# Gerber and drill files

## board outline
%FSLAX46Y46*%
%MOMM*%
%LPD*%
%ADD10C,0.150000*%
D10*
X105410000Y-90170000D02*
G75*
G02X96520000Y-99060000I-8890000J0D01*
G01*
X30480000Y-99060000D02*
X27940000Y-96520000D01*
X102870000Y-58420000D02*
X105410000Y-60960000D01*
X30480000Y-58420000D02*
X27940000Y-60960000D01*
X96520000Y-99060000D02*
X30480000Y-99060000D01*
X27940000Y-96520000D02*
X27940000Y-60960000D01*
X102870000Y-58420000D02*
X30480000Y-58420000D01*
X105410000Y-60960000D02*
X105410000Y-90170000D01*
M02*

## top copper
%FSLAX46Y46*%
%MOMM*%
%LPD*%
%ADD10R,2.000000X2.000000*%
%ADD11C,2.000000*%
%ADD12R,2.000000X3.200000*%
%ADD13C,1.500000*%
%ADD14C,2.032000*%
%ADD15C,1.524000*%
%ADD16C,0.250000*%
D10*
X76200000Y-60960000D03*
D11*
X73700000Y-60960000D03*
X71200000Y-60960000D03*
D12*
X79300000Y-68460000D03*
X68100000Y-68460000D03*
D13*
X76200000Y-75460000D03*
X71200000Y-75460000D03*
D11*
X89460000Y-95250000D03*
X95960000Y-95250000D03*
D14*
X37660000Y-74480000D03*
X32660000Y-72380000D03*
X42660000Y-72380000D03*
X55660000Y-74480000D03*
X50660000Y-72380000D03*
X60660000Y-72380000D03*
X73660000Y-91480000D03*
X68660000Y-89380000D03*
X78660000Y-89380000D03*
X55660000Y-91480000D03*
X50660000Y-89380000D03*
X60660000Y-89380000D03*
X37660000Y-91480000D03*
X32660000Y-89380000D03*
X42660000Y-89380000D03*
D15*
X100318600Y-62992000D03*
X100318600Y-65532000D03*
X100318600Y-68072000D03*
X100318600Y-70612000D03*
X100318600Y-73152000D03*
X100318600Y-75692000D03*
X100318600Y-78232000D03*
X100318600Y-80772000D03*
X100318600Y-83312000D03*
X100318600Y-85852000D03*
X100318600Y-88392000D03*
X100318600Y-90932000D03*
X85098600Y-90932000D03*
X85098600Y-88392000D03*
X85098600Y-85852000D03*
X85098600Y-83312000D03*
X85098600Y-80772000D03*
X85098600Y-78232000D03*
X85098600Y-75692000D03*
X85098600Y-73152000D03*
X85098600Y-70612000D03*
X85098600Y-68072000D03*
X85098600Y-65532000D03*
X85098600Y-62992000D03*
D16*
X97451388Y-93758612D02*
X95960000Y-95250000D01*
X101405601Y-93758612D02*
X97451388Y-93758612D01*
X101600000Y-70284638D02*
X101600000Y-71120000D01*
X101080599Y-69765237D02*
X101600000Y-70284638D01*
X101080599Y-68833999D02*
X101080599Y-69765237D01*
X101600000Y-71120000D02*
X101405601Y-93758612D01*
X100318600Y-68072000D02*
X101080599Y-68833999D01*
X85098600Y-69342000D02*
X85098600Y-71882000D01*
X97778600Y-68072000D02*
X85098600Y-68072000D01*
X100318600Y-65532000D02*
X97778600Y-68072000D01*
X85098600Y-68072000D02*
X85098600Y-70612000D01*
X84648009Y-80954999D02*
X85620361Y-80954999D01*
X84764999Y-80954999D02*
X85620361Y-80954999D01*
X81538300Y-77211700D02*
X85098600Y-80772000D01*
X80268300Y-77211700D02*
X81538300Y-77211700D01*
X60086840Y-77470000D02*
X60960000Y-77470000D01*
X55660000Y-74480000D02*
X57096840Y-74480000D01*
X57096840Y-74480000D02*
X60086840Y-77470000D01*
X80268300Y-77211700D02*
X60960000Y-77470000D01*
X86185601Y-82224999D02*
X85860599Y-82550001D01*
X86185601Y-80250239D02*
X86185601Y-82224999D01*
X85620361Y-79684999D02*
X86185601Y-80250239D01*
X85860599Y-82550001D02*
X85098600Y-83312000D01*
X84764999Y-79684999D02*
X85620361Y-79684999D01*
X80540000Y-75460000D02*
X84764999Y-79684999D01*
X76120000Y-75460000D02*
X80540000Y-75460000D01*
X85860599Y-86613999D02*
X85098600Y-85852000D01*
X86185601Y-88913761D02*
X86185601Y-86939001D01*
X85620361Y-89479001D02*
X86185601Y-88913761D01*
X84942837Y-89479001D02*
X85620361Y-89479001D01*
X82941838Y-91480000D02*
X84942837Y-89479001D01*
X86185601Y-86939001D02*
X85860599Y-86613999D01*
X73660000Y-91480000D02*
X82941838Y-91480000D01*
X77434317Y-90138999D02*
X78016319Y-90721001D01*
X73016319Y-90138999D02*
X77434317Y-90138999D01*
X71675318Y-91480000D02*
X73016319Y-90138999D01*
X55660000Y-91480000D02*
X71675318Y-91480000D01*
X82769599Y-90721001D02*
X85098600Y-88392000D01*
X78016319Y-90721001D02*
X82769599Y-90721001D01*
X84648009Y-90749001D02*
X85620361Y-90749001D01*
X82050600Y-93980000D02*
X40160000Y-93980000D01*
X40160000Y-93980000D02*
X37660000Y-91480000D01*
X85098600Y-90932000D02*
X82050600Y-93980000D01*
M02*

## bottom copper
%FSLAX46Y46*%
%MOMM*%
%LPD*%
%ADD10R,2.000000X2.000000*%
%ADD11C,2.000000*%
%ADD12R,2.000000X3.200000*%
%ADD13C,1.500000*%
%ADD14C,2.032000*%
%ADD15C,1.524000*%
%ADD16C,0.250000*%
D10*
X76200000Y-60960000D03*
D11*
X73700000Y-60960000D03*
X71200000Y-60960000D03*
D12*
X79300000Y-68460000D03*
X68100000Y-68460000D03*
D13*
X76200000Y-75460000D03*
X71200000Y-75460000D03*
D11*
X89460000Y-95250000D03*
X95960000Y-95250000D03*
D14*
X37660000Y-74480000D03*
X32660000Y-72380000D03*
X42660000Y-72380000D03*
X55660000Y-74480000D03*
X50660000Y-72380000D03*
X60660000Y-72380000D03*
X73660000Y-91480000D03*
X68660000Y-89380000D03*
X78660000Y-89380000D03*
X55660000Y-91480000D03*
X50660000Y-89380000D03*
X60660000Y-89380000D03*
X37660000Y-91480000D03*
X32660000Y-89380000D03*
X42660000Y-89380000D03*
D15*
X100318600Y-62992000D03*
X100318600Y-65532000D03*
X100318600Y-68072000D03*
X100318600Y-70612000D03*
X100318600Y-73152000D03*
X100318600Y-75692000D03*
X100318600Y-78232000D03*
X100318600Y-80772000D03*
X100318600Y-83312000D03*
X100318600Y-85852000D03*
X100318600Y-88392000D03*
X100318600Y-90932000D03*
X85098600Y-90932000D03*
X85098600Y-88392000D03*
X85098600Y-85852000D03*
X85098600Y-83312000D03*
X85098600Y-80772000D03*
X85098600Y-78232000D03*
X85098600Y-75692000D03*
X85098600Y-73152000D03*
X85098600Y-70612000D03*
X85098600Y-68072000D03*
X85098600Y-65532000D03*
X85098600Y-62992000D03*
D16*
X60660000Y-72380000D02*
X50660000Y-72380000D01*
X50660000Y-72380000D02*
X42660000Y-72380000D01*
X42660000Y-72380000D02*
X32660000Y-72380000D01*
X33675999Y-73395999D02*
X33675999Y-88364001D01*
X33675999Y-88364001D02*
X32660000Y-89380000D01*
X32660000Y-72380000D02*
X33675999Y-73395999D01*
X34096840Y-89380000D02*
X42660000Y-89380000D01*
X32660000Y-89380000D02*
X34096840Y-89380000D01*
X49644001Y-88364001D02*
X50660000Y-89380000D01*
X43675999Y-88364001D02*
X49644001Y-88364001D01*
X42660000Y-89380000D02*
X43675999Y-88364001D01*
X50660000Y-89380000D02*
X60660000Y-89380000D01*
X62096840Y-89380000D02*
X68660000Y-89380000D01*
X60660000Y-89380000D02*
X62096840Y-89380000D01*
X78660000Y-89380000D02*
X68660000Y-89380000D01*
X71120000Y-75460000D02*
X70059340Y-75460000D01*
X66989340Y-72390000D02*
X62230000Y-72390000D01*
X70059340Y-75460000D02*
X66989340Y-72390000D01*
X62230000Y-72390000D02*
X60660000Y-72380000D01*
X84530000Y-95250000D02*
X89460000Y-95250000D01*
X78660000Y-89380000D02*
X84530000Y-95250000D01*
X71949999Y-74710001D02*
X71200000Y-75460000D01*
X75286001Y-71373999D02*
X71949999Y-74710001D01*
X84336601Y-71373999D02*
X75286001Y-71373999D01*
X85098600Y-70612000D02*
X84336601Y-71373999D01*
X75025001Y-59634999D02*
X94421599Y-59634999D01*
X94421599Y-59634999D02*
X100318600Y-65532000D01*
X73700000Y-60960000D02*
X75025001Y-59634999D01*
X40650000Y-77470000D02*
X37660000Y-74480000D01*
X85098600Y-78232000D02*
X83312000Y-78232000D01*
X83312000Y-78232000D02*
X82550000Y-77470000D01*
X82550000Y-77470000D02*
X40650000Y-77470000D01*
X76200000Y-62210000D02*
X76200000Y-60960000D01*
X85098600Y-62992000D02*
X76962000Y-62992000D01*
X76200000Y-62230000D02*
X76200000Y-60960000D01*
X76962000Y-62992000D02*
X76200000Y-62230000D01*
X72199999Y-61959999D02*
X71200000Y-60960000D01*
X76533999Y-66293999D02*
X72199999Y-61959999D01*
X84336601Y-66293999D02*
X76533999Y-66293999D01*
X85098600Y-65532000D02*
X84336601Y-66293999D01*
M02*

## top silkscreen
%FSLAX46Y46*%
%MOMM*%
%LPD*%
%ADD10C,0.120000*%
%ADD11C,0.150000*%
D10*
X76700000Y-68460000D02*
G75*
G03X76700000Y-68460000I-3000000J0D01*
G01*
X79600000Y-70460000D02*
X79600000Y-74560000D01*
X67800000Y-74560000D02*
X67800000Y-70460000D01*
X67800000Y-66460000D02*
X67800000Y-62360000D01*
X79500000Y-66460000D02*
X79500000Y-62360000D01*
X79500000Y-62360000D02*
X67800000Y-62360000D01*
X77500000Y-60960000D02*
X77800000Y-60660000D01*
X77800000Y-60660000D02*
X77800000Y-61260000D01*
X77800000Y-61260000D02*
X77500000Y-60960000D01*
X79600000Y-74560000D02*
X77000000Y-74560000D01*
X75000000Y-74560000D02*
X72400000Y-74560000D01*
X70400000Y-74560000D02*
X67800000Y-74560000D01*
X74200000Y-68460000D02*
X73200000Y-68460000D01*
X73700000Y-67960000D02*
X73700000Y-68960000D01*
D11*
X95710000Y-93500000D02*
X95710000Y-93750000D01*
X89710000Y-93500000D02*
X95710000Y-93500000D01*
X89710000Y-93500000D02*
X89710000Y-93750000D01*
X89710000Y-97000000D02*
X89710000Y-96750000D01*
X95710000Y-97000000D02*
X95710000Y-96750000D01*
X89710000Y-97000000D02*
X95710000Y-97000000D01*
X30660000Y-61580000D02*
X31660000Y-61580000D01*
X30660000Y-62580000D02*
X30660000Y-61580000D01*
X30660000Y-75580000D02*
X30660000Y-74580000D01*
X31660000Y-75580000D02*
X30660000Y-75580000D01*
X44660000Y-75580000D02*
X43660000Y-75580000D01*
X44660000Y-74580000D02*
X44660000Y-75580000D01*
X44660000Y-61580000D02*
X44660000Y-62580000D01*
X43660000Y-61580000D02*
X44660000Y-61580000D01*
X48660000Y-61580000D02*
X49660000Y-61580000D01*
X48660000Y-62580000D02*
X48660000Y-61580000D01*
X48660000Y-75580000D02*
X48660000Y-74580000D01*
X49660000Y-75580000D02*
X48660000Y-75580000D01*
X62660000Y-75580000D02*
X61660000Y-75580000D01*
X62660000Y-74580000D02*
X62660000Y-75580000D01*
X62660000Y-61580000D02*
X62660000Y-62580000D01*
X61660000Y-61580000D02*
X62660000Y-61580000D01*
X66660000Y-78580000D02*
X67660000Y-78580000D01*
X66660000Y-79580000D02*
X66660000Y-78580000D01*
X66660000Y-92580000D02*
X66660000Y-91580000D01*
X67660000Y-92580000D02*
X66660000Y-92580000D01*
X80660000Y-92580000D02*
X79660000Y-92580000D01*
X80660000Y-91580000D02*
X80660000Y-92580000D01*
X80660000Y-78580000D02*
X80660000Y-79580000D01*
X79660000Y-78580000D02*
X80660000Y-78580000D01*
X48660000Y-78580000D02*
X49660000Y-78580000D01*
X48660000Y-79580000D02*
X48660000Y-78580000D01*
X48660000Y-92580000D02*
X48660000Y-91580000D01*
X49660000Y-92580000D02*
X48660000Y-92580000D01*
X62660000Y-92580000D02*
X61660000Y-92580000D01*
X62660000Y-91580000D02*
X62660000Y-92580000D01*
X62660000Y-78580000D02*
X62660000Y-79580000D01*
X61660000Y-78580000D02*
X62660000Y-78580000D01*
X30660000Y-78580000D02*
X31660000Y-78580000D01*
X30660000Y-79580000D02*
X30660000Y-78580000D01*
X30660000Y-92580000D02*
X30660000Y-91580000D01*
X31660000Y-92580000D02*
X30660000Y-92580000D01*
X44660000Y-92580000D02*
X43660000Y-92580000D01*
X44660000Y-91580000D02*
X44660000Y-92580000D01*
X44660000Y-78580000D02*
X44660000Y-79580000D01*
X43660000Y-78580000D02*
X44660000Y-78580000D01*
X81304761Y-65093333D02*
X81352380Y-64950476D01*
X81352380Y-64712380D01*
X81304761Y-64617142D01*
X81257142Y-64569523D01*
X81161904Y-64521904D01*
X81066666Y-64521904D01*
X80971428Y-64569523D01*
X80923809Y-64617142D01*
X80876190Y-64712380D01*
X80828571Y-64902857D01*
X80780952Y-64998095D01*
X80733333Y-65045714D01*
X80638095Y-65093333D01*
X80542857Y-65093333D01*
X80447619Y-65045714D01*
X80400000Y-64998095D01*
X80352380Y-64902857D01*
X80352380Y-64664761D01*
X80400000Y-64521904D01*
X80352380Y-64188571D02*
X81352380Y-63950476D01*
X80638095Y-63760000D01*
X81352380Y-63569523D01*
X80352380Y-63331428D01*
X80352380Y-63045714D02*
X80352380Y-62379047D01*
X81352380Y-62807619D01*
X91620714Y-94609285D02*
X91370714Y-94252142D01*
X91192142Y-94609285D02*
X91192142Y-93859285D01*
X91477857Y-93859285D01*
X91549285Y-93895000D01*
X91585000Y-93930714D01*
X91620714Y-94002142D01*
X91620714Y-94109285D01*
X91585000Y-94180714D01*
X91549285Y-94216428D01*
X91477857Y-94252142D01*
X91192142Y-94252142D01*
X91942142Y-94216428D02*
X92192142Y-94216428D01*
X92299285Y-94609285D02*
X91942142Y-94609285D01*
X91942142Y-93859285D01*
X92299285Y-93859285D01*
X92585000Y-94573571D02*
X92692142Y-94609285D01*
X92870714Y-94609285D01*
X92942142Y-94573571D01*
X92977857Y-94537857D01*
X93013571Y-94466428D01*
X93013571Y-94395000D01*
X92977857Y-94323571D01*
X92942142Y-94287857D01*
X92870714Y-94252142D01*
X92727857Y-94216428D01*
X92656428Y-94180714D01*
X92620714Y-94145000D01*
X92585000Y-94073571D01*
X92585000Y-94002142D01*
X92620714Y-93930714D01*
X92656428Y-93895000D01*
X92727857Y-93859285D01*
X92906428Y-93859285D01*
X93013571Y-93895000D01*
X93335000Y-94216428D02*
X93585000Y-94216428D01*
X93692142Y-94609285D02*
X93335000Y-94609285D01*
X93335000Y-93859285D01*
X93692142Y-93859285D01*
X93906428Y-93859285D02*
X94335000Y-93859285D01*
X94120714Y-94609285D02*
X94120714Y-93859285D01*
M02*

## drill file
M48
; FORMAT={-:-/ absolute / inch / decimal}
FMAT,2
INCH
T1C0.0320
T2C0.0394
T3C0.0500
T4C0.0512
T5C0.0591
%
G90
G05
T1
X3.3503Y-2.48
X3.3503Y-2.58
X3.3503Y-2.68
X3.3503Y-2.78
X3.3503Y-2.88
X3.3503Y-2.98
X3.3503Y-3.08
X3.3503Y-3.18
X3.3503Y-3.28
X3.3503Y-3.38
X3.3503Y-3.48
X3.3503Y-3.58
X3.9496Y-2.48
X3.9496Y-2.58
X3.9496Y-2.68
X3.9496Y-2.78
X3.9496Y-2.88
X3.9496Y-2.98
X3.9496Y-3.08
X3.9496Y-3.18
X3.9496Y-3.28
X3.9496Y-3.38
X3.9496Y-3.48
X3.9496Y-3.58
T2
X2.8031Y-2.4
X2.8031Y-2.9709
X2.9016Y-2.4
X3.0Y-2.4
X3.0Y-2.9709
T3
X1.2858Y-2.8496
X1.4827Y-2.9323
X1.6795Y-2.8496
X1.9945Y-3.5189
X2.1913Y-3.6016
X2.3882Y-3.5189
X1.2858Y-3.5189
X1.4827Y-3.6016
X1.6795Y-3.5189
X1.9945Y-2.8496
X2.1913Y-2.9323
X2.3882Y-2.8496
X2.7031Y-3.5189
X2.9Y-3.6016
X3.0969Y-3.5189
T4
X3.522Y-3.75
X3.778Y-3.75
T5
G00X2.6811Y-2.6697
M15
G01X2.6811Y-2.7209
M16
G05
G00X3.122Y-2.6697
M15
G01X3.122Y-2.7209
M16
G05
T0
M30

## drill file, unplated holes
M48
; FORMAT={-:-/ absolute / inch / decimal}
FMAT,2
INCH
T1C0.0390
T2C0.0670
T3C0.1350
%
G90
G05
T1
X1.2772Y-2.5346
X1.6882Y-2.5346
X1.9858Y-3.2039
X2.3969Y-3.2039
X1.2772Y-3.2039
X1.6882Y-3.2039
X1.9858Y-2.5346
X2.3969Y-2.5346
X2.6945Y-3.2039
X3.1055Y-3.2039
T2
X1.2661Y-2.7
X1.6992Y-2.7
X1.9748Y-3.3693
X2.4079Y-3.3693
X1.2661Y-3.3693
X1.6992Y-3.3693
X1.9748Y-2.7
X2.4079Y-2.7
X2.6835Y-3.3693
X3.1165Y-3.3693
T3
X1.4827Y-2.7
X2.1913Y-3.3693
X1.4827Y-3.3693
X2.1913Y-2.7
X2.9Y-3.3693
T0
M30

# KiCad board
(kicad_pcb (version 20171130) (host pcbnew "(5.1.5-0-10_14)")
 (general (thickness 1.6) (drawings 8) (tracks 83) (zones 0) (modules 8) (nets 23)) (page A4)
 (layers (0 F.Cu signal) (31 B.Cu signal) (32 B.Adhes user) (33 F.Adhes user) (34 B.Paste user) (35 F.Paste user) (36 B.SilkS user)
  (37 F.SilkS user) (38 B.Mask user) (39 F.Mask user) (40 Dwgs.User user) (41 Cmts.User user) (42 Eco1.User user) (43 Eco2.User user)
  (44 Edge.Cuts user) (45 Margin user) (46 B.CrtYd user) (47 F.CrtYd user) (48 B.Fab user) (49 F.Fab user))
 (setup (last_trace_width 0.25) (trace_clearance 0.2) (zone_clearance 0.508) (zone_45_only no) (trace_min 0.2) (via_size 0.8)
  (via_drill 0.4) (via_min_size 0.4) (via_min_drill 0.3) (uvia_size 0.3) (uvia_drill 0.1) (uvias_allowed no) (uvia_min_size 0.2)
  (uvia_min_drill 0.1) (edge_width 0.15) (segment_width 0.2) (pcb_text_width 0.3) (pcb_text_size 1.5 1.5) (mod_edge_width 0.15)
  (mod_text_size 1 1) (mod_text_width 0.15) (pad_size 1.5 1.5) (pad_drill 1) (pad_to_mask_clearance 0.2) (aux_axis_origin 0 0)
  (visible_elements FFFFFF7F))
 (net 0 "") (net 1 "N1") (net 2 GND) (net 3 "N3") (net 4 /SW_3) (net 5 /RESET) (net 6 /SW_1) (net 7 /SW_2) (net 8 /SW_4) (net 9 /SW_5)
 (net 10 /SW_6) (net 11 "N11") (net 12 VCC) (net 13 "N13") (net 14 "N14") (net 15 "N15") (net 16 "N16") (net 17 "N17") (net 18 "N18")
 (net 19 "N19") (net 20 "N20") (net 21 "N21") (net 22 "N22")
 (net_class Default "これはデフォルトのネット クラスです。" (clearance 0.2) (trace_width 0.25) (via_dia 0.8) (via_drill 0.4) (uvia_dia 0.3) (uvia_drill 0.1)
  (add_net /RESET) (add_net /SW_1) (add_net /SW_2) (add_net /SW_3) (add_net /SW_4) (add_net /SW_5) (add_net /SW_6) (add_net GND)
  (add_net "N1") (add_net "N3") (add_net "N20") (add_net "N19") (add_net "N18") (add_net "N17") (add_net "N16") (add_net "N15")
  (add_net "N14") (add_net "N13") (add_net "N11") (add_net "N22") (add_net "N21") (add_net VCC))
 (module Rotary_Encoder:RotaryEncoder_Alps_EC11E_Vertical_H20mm (layer F.Cu) (at 76.2 60.96 270)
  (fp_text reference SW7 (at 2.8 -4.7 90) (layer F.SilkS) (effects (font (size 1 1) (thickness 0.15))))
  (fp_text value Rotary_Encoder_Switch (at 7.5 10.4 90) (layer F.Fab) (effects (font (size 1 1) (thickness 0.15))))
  (fp_circle (center 7.5 2.5) (end 10.5 2.5) (layer F.SilkS) (width 0.12))
  (fp_line (start 9.5 -3.4) (end 13.6 -3.4) (layer F.SilkS) (width 0.12))
  (fp_line (start 13.6 8.4) (end 9.5 8.4) (layer F.SilkS) (width 0.12))
  (fp_line (start 5.5 8.4) (end 1.4 8.4) (layer F.SilkS) (width 0.12))
  (fp_line (start 5.5 -3.3) (end 1.4 -3.3) (layer F.SilkS) (width 0.12))
  (fp_line (start 1.4 -3.3) (end 1.4 8.4) (layer F.SilkS) (width 0.12))
  (fp_line (start 0 -1.3) (end -0.3 -1.6) (layer F.SilkS) (width 0.12))
  (fp_line (start -0.3 -1.6) (end 0.3 -1.6) (layer F.SilkS) (width 0.12))
  (fp_line (start 0.3 -1.6) (end 0 -1.3) (layer F.SilkS) (width 0.12))
  (fp_line (start 13.6 -3.4) (end 13.6 -0.8) (layer F.SilkS) (width 0.12))
  (fp_line (start 13.6 1.2) (end 13.6 3.8) (layer F.SilkS) (width 0.12))
  (fp_line (start 13.6 5.8) (end 13.6 8.4) (layer F.SilkS) (width 0.12))
  (fp_line (start 7.5 2) (end 7.5 3) (layer F.SilkS) (width 0.12))
  (fp_line (start 7 2.5) (end 8 2.5) (layer F.SilkS) (width 0.12))
  (pad A thru_hole rect (at 0 0 270) (size 2 2) (drill 1) (layers *.Cu *.Mask) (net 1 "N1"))
  (pad C thru_hole circle (at 0 2.5 270) (size 2 2) (drill 1) (layers *.Cu *.Mask) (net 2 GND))
  (pad B thru_hole circle (at 0 5 270) (size 2 2) (drill 1) (layers *.Cu *.Mask) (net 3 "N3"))
  (pad MP thru_hole rect (at 7.5 -3.1 270) (size 3.2 2) (drill oval 2.8 1.5) (layers *.Cu *.Mask))
  (pad MP thru_hole rect (at 7.5 8.1 270) (size 3.2 2) (drill oval 2.8 1.5) (layers *.Cu *.Mask))
  (pad "" thru_hole circle (at 14.5 0 270) (size 1.5 1.5) (drill 1) (layers *.Cu *.Mask) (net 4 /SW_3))
  (pad "" thru_hole circle (at 14.5 5 270) (size 1.5 1.5) (drill 1) (layers *.Cu *.Mask) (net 2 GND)))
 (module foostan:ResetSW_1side (layer F.Cu) (at 92.71 95.25)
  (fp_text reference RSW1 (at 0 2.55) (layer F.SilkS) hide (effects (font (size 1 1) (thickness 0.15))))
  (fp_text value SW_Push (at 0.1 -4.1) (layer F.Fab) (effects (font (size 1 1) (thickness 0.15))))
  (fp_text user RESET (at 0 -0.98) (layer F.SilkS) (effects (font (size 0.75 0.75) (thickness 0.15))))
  (fp_line (start 3 -1.75) (end 3 -1.5) (layer F.SilkS) (width 0.15))
  (fp_line (start -3 -1.75) (end 3 -1.75) (layer F.SilkS) (width 0.15))
  (fp_line (start -3 -1.75) (end -3 -1.5) (layer F.SilkS) (width 0.15))
  (fp_line (start -3 1.75) (end -3 1.5) (layer F.SilkS) (width 0.15))
  (fp_line (start 3 1.75) (end 3 1.5) (layer F.SilkS) (width 0.15))
  (fp_line (start -3 1.75) (end 3 1.75) (layer F.SilkS) (width 0.15))
  (pad 2 thru_hole circle (at -3.25 0) (size 2 2) (drill 1.3) (layers *.Cu F.SilkS B.Mask) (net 2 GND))
  (pad 1 thru_hole circle (at 3.25 0) (size 2 2) (drill 1.3) (layers *.Cu F.SilkS B.Mask) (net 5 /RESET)))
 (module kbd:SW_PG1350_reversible (layer F.Cu) (at 37.66 68.58)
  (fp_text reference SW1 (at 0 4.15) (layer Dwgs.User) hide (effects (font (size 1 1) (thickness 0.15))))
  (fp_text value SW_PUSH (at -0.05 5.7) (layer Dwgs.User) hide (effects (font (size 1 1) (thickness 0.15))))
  (fp_line (start -7 -7) (end -6 -7) (layer F.SilkS) (width 0.15))
  (fp_line (start -7 -6) (end -7 -7) (layer F.SilkS) (width 0.15))
  (fp_line (start -7 7) (end -7 6) (layer F.SilkS) (width 0.15))
  (fp_line (start -6 7) (end -7 7) (layer F.SilkS) (width 0.15)) (fp_line (start 7 7) (end 6 7) (layer F.SilkS) (width 0.15))
  (fp_line (start 7 6) (end 7 7) (layer F.SilkS) (width 0.15))
  (fp_line (start 7 -7) (end 7 -6) (layer F.SilkS) (width 0.15))
  (fp_line (start 6 -7) (end 7 -7) (layer F.SilkS) (width 0.15))
  (pad "" np_thru_hole circle (at -5.5 0) (size 1.7018 1.7018) (drill 1.7018) (layers *.Cu *.Mask))
  (pad "" np_thru_hole circle (at 5.5 0) (size 1.7018 1.7018) (drill 1.7018) (layers *.Cu *.Mask))
  (pad "" np_thru_hole circle (at 5.22 -4.2) (size 0.9906 0.9906) (drill 0.9906) (layers *.Cu *.Mask))
  (pad 1 thru_hole circle (at 0 5.9) (size 2.032 2.032) (drill 1.27) (layers *.Cu *.Mask) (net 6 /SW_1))
  (pad 2 thru_hole circle (at -5 3.8) (size 2.032 2.032) (drill 1.27) (layers *.Cu *.Mask) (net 2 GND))
  (pad "" np_thru_hole circle (at 0 0) (size 3.429 3.429) (drill 3.429) (layers *.Cu *.Mask))
  (pad 2 thru_hole circle (at 5 3.8) (size 2.032 2.032) (drill 1.27) (layers *.Cu *.Mask) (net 2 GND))
  (pad "" np_thru_hole circle (at -5.22 -4.2) (size 0.9906 0.9906) (drill 0.9906) (layers *.Cu *.Mask)))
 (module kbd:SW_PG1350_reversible (layer F.Cu) (at 55.66 68.58)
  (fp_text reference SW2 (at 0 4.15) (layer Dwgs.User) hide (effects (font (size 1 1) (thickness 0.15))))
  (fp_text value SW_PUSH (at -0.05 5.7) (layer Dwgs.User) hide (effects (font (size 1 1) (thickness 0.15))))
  (fp_line (start -7 -7) (end -6 -7) (layer F.SilkS) (width 0.15))
  (fp_line (start -7 -6) (end -7 -7) (layer F.SilkS) (width 0.15))
  (fp_line (start -7 7) (end -7 6) (layer F.SilkS) (width 0.15))
  (fp_line (start -6 7) (end -7 7) (layer F.SilkS) (width 0.15)) (fp_line (start 7 7) (end 6 7) (layer F.SilkS) (width 0.15))
  (fp_line (start 7 6) (end 7 7) (layer F.SilkS) (width 0.15))
  (fp_line (start 7 -7) (end 7 -6) (layer F.SilkS) (width 0.15))
  (fp_line (start 6 -7) (end 7 -7) (layer F.SilkS) (width 0.15))
  (pad "" np_thru_hole circle (at -5.5 0) (size 1.7018 1.7018) (drill 1.7018) (layers *.Cu *.Mask))
  (pad "" np_thru_hole circle (at 5.5 0) (size 1.7018 1.7018) (drill 1.7018) (layers *.Cu *.Mask))
  (pad "" np_thru_hole circle (at 5.22 -4.2) (size 0.9906 0.9906) (drill 0.9906) (layers *.Cu *.Mask))
  (pad 1 thru_hole circle (at 0 5.9) (size 2.032 2.032) (drill 1.27) (layers *.Cu *.Mask) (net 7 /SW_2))
  (pad 2 thru_hole circle (at -5 3.8) (size 2.032 2.032) (drill 1.27) (layers *.Cu *.Mask) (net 2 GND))
  (pad "" np_thru_hole circle (at 0 0) (size 3.429 3.429) (drill 3.429) (layers *.Cu *.Mask))
  (pad 2 thru_hole circle (at 5 3.8) (size 2.032 2.032) (drill 1.27) (layers *.Cu *.Mask) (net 2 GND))
  (pad "" np_thru_hole circle (at -5.22 -4.2) (size 0.9906 0.9906) (drill 0.9906) (layers *.Cu *.Mask)))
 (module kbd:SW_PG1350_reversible (layer F.Cu) (at 73.66 85.58)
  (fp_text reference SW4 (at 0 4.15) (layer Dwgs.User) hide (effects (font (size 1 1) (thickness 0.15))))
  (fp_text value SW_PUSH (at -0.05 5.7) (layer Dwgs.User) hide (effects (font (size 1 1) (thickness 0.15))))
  (fp_line (start -7 -7) (end -6 -7) (layer F.SilkS) (width 0.15))
  (fp_line (start -7 -6) (end -7 -7) (layer F.SilkS) (width 0.15))
  (fp_line (start -7 7) (end -7 6) (layer F.SilkS) (width 0.15))
  (fp_line (start -6 7) (end -7 7) (layer F.SilkS) (width 0.15)) (fp_line (start 7 7) (end 6 7) (layer F.SilkS) (width 0.15))
  (fp_line (start 7 6) (end 7 7) (layer F.SilkS) (width 0.15))
  (fp_line (start 7 -7) (end 7 -6) (layer F.SilkS) (width 0.15))
  (fp_line (start 6 -7) (end 7 -7) (layer F.SilkS) (width 0.15))
  (pad "" np_thru_hole circle (at -5.5 0) (size 1.7018 1.7018) (drill 1.7018) (layers *.Cu *.Mask))
  (pad "" np_thru_hole circle (at 5.5 0) (size 1.7018 1.7018) (drill 1.7018) (layers *.Cu *.Mask))
  (pad "" np_thru_hole circle (at 5.22 -4.2) (size 0.9906 0.9906) (drill 0.9906) (layers *.Cu *.Mask))
  (pad 1 thru_hole circle (at 0 5.9) (size 2.032 2.032) (drill 1.27) (layers *.Cu *.Mask) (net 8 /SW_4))
  (pad 2 thru_hole circle (at -5 3.8) (size 2.032 2.032) (drill 1.27) (layers *.Cu *.Mask) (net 2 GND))
  (pad "" np_thru_hole circle (at 0 0) (size 3.429 3.429) (drill 3.429) (layers *.Cu *.Mask))
  (pad 2 thru_hole circle (at 5 3.8) (size 2.032 2.032) (drill 1.27) (layers *.Cu *.Mask) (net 2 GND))
  (pad "" np_thru_hole circle (at -5.22 -4.2) (size 0.9906 0.9906) (drill 0.9906) (layers *.Cu *.Mask)))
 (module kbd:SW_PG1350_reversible (layer F.Cu) (at 55.66 85.58)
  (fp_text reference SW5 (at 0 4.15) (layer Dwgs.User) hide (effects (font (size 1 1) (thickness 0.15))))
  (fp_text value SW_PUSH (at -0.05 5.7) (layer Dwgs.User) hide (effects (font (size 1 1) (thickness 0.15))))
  (fp_line (start -7 -7) (end -6 -7) (layer F.SilkS) (width 0.15))
  (fp_line (start -7 -6) (end -7 -7) (layer F.SilkS) (width 0.15))
  (fp_line (start -7 7) (end -7 6) (layer F.SilkS) (width 0.15))
  (fp_line (start -6 7) (end -7 7) (layer F.SilkS) (width 0.15)) (fp_line (start 7 7) (end 6 7) (layer F.SilkS) (width 0.15))
  (fp_line (start 7 6) (end 7 7) (layer F.SilkS) (width 0.15))
  (fp_line (start 7 -7) (end 7 -6) (layer F.SilkS) (width 0.15))
  (fp_line (start 6 -7) (end 7 -7) (layer F.SilkS) (width 0.15))
  (pad "" np_thru_hole circle (at -5.5 0) (size 1.7018 1.7018) (drill 1.7018) (layers *.Cu *.Mask))
  (pad "" np_thru_hole circle (at 5.5 0) (size 1.7018 1.7018) (drill 1.7018) (layers *.Cu *.Mask))
  (pad "" np_thru_hole circle (at 5.22 -4.2) (size 0.9906 0.9906) (drill 0.9906) (layers *.Cu *.Mask))
  (pad 1 thru_hole circle (at 0 5.9) (size 2.032 2.032) (drill 1.27) (layers *.Cu *.Mask) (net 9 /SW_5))
  (pad 2 thru_hole circle (at -5 3.8) (size 2.032 2.032) (drill 1.27) (layers *.Cu *.Mask) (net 2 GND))
  (pad "" np_thru_hole circle (at 0 0) (size 3.429 3.429) (drill 3.429) (layers *.Cu *.Mask))
  (pad 2 thru_hole circle (at 5 3.8) (size 2.032 2.032) (drill 1.27) (layers *.Cu *.Mask) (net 2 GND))
  (pad "" np_thru_hole circle (at -5.22 -4.2) (size 0.9906 0.9906) (drill 0.9906) (layers *.Cu *.Mask)))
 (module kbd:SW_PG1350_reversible (layer F.Cu) (at 37.66 85.58)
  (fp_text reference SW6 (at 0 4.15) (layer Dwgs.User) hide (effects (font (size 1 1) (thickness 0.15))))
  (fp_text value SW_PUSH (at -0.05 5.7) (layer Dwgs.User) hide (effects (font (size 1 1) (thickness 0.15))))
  (fp_line (start -7 -7) (end -6 -7) (layer F.SilkS) (width 0.15))
  (fp_line (start -7 -6) (end -7 -7) (layer F.SilkS) (width 0.15))
  (fp_line (start -7 7) (end -7 6) (layer F.SilkS) (width 0.15))
  (fp_line (start -6 7) (end -7 7) (layer F.SilkS) (width 0.15)) (fp_line (start 7 7) (end 6 7) (layer F.SilkS) (width 0.15))
  (fp_line (start 7 6) (end 7 7) (layer F.SilkS) (width 0.15))
  (fp_line (start 7 -7) (end 7 -6) (layer F.SilkS) (width 0.15))
  (fp_line (start 6 -7) (end 7 -7) (layer F.SilkS) (width 0.15))
  (pad "" np_thru_hole circle (at -5.5 0) (size 1.7018 1.7018) (drill 1.7018) (layers *.Cu *.Mask))
  (pad "" np_thru_hole circle (at 5.5 0) (size 1.7018 1.7018) (drill 1.7018) (layers *.Cu *.Mask))
  (pad "" np_thru_hole circle (at 5.22 -4.2) (size 0.9906 0.9906) (drill 0.9906) (layers *.Cu *.Mask))
  (pad 1 thru_hole circle (at 0 5.9) (size 2.032 2.032) (drill 1.27) (layers *.Cu *.Mask) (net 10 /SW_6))
  (pad 2 thru_hole circle (at -5 3.8) (size 2.032 2.032) (drill 1.27) (layers *.Cu *.Mask) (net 2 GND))
  (pad "" np_thru_hole circle (at 0 0) (size 3.429 3.429) (drill 3.429) (layers *.Cu *.Mask))
  (pad 2 thru_hole circle (at 5 3.8) (size 2.032 2.032) (drill 1.27) (layers *.Cu *.Mask) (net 2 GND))
  (pad "" np_thru_hole circle (at -5.22 -4.2) (size 0.9906 0.9906) (drill 0.9906) (layers *.Cu *.Mask)))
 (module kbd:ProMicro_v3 (layer B.Cu) (at 92.71 77.47 180)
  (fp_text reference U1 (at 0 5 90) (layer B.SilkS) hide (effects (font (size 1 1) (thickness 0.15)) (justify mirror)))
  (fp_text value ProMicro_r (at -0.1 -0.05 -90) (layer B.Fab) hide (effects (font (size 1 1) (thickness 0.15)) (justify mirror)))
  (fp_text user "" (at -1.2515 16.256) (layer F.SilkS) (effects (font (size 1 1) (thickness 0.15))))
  (pad 24 thru_hole circle (at -7.6086 14.478 180) (size 1.524 1.524) (drill 0.8128) (layers *.Cu B.SilkS F.Mask) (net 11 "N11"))
  (pad 23 thru_hole circle (at -7.6086 11.938 180) (size 1.524 1.524) (drill 0.8128) (layers *.Cu B.SilkS F.Mask) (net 2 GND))
  (pad 22 thru_hole circle (at -7.6086 9.398 180) (size 1.524 1.524) (drill 0.8128) (layers *.Cu B.SilkS F.Mask) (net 5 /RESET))
  (pad 21 thru_hole circle (at -7.6086 6.858 180) (size 1.524 1.524) (drill 0.8128) (layers *.Cu B.SilkS F.Mask) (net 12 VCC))
  (pad 20 thru_hole circle (at -7.6086 4.318 180) (size 1.524 1.524) (drill 0.8128) (layers *.Cu B.SilkS F.Mask) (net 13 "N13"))
  (pad 19 thru_hole circle (at -7.6086 1.778 180) (size 1.524 1.524) (drill 0.8128) (layers *.Cu B.SilkS F.Mask) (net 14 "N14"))
  (pad 18 thru_hole circle (at -7.6086 -0.762 180) (size 1.524 1.524) (drill 0.8128) (layers *.Cu B.SilkS F.Mask) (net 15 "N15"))
  (pad 17 thru_hole circle (at -7.6086 -3.302 180) (size 1.524 1.524) (drill 0.8128) (layers *.Cu B.SilkS F.Mask) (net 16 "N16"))
  (pad 16 thru_hole circle (at -7.6086 -5.842 180) (size 1.524 1.524) (drill 0.8128) (layers *.Cu B.SilkS F.Mask) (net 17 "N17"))
  (pad 15 thru_hole circle (at -7.6086 -8.382 180) (size 1.524 1.524) (drill 0.8128) (layers *.Cu B.SilkS F.Mask) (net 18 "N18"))
  (pad 14 thru_hole circle (at -7.6086 -10.922 180) (size 1.524 1.524) (drill 0.8128) (layers *.Cu B.SilkS F.Mask) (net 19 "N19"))
  (pad 13 thru_hole circle (at -7.6086 -13.462 180) (size 1.524 1.524) (drill 0.8128) (layers *.Cu B.SilkS F.Mask) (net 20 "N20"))
  (pad 12 thru_hole circle (at 7.6114 -13.462 180) (size 1.524 1.524) (drill 0.8128) (layers *.Cu B.SilkS F.Mask) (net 10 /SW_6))
  (pad 11 thru_hole circle (at 7.6114 -10.922 180) (size 1.524 1.524) (drill 0.8128) (layers *.Cu B.SilkS F.Mask) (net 9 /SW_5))
  (pad 10 thru_hole circle (at 7.6114 -8.382 180) (size 1.524 1.524) (drill 0.8128) (layers *.Cu B.SilkS F.Mask) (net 8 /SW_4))
  (pad 9 thru_hole circle (at 7.6114 -5.842 180) (size 1.524 1.524) (drill 0.8128) (layers *.Cu B.SilkS F.Mask) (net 4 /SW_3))
  (pad 8 thru_hole circle (at 7.6114 -3.302 180) (size 1.524 1.524) (drill 0.8128) (layers *.Cu B.SilkS F.Mask) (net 7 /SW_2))
  (pad 7 thru_hole circle (at 7.6114 -0.762 180) (size 1.524 1.524) (drill 0.8128) (layers *.Cu B.SilkS F.Mask) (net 6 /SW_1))
  (pad 6 thru_hole circle (at 7.6114 1.778 180) (size 1.524 1.524) (drill 0.8128) (layers *.Cu B.SilkS F.Mask) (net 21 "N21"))
  (pad 5 thru_hole circle (at 7.6114 4.318 180) (size 1.524 1.524) (drill 0.8128) (layers *.Cu B.SilkS F.Mask) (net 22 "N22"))
  (pad 4 thru_hole circle (at 7.6114 6.858 180) (size 1.524 1.524) (drill 0.8128) (layers *.Cu B.SilkS F.Mask) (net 2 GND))
  (pad 3 thru_hole circle (at 7.6114 9.398 180) (size 1.524 1.524) (drill 0.8128) (layers *.Cu B.SilkS F.Mask) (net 2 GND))
  (pad 2 thru_hole circle (at 7.6114 11.938 180) (size 1.524 1.524) (drill 0.8128) (layers *.Cu B.SilkS F.Mask) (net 3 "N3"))
  (pad 1 thru_hole circle (at 7.6114 14.478 180) (size 1.524 1.524) (drill 0.8128) (layers *.Cu B.SilkS F.Mask) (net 1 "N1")))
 (gr_arc (start 96.52 90.17) (end 96.52 99.06) (angle -90) (layer Edge.Cuts) (width 0.15))
 (gr_line (start 30.48 99.06) (end 27.94 96.52) (layer Edge.Cuts) (width 0.15))
 (gr_line (start 102.87 58.42) (end 105.41 60.96) (layer Edge.Cuts) (width 0.15))
 (gr_line (start 30.48 58.42) (end 27.94 60.96) (layer Edge.Cuts) (width 0.15))
 (gr_line (start 96.52 99.06) (end 30.48 99.06) (layer Edge.Cuts) (width 0.15))
 (gr_line (start 27.94 96.52) (end 27.94 60.96) (layer Edge.Cuts) (width 0.15))
 (gr_line (start 102.87 58.42) (end 30.48 58.42) (layer Edge.Cuts) (width 0.15))
 (gr_line (start 105.41 60.96) (end 105.41 90.17) (layer Edge.Cuts) (width 0.15))
 (segment (start 97.451388 93.758612) (end 95.96 95.25) (width 0.25) (layer F.Cu) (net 5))
 (segment (start 101.405601 93.758612) (end 97.451388 93.758612) (width 0.25) (layer F.Cu) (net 5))
 (segment (start 101.6 70.284638) (end 101.6 71.12) (width 0.25) (layer F.Cu) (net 5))
 (segment (start 101.080599 69.765237) (end 101.6 70.284638) (width 0.25) (layer F.Cu) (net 5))
 (segment (start 101.080599 68.833999) (end 101.080599 69.765237) (width 0.25) (layer F.Cu) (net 5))
 (segment (start 101.6 71.12) (end 101.405601 93.758612) (width 0.25) (layer F.Cu) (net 5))
 (segment (start 100.3186 68.072) (end 101.080599 68.833999) (width 0.25) (layer F.Cu) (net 5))
 (segment (start 60.66 72.38) (end 50.66 72.38) (width 0.25) (layer B.Cu) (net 2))
 (segment (start 50.66 72.38) (end 42.66 72.38) (width 0.25) (layer B.Cu) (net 2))
 (segment (start 42.66 72.38) (end 32.66 72.38) (width 0.25) (layer B.Cu) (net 2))
 (segment (start 33.675999 73.395999) (end 33.675999 88.364001) (width 0.25) (layer B.Cu) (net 2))
 (segment (start 33.675999 88.364001) (end 32.66 89.38) (width 0.25) (layer B.Cu) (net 2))
 (segment (start 32.66 72.38) (end 33.675999 73.395999) (width 0.25) (layer B.Cu) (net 2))
 (segment (start 34.09684 89.38) (end 42.66 89.38) (width 0.25) (layer B.Cu) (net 2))
 (segment (start 32.66 89.38) (end 34.09684 89.38) (width 0.25) (layer B.Cu) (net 2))
 (segment (start 49.644001 88.364001) (end 50.66 89.38) (width 0.25) (layer B.Cu) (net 2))
 (segment (start 43.675999 88.364001) (end 49.644001 88.364001) (width 0.25) (layer B.Cu) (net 2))
 (segment (start 42.66 89.38) (end 43.675999 88.364001) (width 0.25) (layer B.Cu) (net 2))
 (segment (start 50.66 89.38) (end 60.66 89.38) (width 0.25) (layer B.Cu) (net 2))
 (segment (start 62.09684 89.38) (end 68.66 89.38) (width 0.25) (layer B.Cu) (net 2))
 (segment (start 60.66 89.38) (end 62.09684 89.38) (width 0.25) (layer B.Cu) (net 2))
 (segment (start 78.66 89.38) (end 68.66 89.38) (width 0.25) (layer B.Cu) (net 2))
 (segment (start 85.0986 69.342) (end 85.0986 71.882) (width 0.25) (layer F.Cu) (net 2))
 (segment (start 71.12 75.46) (end 70.05934 75.46) (width 0.25) (layer B.Cu) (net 2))
 (segment (start 66.98934 72.39) (end 62.23 72.39) (width 0.25) (layer B.Cu) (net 2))
 (segment (start 70.05934 75.46) (end 66.98934 72.39) (width 0.25) (layer B.Cu) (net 2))
 (segment (start 62.23 72.39) (end 60.66 72.38) (width 0.25) (layer B.Cu) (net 2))
 (segment (start 84.53 95.25) (end 89.46 95.25) (width 0.25) (layer B.Cu) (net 2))
 (segment (start 78.66 89.38) (end 84.53 95.25) (width 0.25) (layer B.Cu) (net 2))
 (segment (start 71.949999 74.710001) (end 71.2 75.46) (width 0.25) (layer B.Cu) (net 2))
 (segment (start 75.286001 71.373999) (end 71.949999 74.710001) (width 0.25) (layer B.Cu) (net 2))
 (segment (start 84.336601 71.373999) (end 75.286001 71.373999) (width 0.25) (layer B.Cu) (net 2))
 (segment (start 85.0986 70.612) (end 84.336601 71.373999) (width 0.25) (layer B.Cu) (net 2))
 (segment (start 97.7786 68.072) (end 85.0986 68.072) (width 0.25) (layer F.Cu) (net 2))
 (segment (start 100.3186 65.532) (end 97.7786 68.072) (width 0.25) (layer F.Cu) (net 2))
 (segment (start 85.0986 68.072) (end 85.0986 70.612) (width 0.25) (layer F.Cu) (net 2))
 (segment (start 75.025001 59.634999) (end 94.421599 59.634999) (width 0.25) (layer B.Cu) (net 2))
 (segment (start 94.421599 59.634999) (end 100.3186 65.532) (width 0.25) (layer B.Cu) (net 2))
 (segment (start 73.7 60.96) (end 75.025001 59.634999) (width 0.25) (layer B.Cu) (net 2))
 (segment (start 40.65 77.47) (end 37.66 74.48) (width 0.25) (layer B.Cu) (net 6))
 (segment (start 85.0986 78.232) (end 83.312 78.232) (width 0.25) (layer B.Cu) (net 6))
 (segment (start 83.312 78.232) (end 82.55 77.47) (width 0.25) (layer B.Cu) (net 6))
 (segment (start 82.55 77.47) (end 40.65 77.47) (width 0.25) (layer B.Cu) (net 6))
 (segment (start 84.648009 80.954999) (end 85.620361 80.954999) (width 0.25) (layer F.Cu) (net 7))
 (segment (start 84.764999 80.954999) (end 85.620361 80.954999) (width 0.25) (layer F.Cu) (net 7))
 (segment (start 81.5383 77.2117) (end 85.0986 80.772) (width 0.25) (layer F.Cu) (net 7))
 (segment (start 80.2683 77.2117) (end 81.5383 77.2117) (width 0.25) (layer F.Cu) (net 7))
 (segment (start 60.08684 77.47) (end 60.96 77.47) (width 0.25) (layer F.Cu) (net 7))
 (segment (start 55.66 74.48) (end 57.09684 74.48) (width 0.25) (layer F.Cu) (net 7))
 (segment (start 57.09684 74.48) (end 60.08684 77.47) (width 0.25) (layer F.Cu) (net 7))
 (segment (start 80.2683 77.2117) (end 60.96 77.47) (width 0.25) (layer F.Cu) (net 7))
 (segment (start 86.185601 82.224999) (end 85.860599 82.550001) (width 0.25) (layer F.Cu) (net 4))
 (segment (start 86.185601 80.250239) (end 86.185601 82.224999) (width 0.25) (layer F.Cu) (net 4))
 (segment (start 85.620361 79.684999) (end 86.185601 80.250239) (width 0.25) (layer F.Cu) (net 4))
 (segment (start 85.860599 82.550001) (end 85.0986 83.312) (width 0.25) (layer F.Cu) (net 4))
 (segment (start 84.764999 79.684999) (end 85.620361 79.684999) (width 0.25) (layer F.Cu) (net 4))
 (segment (start 80.54 75.46) (end 84.764999 79.684999) (width 0.25) (layer F.Cu) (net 4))
 (segment (start 76.12 75.46) (end 80.54 75.46) (width 0.25) (layer F.Cu) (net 4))
 (segment (start 85.860599 86.613999) (end 85.0986 85.852) (width 0.25) (layer F.Cu) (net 8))
 (segment (start 86.185601 88.913761) (end 86.185601 86.939001) (width 0.25) (layer F.Cu) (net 8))
 (segment (start 85.620361 89.479001) (end 86.185601 88.913761) (width 0.25) (layer F.Cu) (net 8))
 (segment (start 84.942837 89.479001) (end 85.620361 89.479001) (width 0.25) (layer F.Cu) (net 8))
 (segment (start 82.941838 91.48) (end 84.942837 89.479001) (width 0.25) (layer F.Cu) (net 8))
 (segment (start 86.185601 86.939001) (end 85.860599 86.613999) (width 0.25) (layer F.Cu) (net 8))
 (segment (start 73.66 91.48) (end 82.941838 91.48) (width 0.25) (layer F.Cu) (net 8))
 (segment (start 77.434317 90.138999) (end 78.016319 90.721001) (width 0.25) (layer F.Cu) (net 9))
 (segment (start 73.016319 90.138999) (end 77.434317 90.138999) (width 0.25) (layer F.Cu) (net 9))
 (segment (start 71.675318 91.48) (end 73.016319 90.138999) (width 0.25) (layer F.Cu) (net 9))
 (segment (start 55.66 91.48) (end 71.675318 91.48) (width 0.25) (layer F.Cu) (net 9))
 (segment (start 82.769599 90.721001) (end 85.0986 88.392) (width 0.25) (layer F.Cu) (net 9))
 (segment (start 78.016319 90.721001) (end 82.769599 90.721001) (width 0.25) (layer F.Cu) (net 9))
 (segment (start 84.648009 90.749001) (end 85.620361 90.749001) (width 0.25) (layer F.Cu) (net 10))
 (segment (start 82.0506 93.98) (end 40.16 93.98) (width 0.25) (layer F.Cu) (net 10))
 (segment (start 40.16 93.98) (end 37.66 91.48) (width 0.25) (layer F.Cu) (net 10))
 (segment (start 85.0986 90.932) (end 82.0506 93.98) (width 0.25) (layer F.Cu) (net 10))
 (segment (start 76.2 62.21) (end 76.2 60.96) (width 0.25) (layer B.Cu) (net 1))
 (segment (start 85.0986 62.992) (end 76.962 62.992) (width 0.25) (layer B.Cu) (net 1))
 (segment (start 76.2 62.23) (end 76.2 60.96) (width 0.25) (layer B.Cu) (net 1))
 (segment (start 76.962 62.992) (end 76.2 62.23) (width 0.25) (layer B.Cu) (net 1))
 (segment (start 72.199999 61.959999) (end 71.2 60.96) (width 0.25) (layer B.Cu) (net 3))
 (segment (start 76.533999 66.293999) (end 72.199999 61.959999) (width 0.25) (layer B.Cu) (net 3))
 (segment (start 84.336601 66.293999) (end 76.533999 66.293999) (width 0.25) (layer B.Cu) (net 3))
 (segment (start 85.0986 65.532) (end 84.336601 66.293999) (width 0.25) (layer B.Cu) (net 3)))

